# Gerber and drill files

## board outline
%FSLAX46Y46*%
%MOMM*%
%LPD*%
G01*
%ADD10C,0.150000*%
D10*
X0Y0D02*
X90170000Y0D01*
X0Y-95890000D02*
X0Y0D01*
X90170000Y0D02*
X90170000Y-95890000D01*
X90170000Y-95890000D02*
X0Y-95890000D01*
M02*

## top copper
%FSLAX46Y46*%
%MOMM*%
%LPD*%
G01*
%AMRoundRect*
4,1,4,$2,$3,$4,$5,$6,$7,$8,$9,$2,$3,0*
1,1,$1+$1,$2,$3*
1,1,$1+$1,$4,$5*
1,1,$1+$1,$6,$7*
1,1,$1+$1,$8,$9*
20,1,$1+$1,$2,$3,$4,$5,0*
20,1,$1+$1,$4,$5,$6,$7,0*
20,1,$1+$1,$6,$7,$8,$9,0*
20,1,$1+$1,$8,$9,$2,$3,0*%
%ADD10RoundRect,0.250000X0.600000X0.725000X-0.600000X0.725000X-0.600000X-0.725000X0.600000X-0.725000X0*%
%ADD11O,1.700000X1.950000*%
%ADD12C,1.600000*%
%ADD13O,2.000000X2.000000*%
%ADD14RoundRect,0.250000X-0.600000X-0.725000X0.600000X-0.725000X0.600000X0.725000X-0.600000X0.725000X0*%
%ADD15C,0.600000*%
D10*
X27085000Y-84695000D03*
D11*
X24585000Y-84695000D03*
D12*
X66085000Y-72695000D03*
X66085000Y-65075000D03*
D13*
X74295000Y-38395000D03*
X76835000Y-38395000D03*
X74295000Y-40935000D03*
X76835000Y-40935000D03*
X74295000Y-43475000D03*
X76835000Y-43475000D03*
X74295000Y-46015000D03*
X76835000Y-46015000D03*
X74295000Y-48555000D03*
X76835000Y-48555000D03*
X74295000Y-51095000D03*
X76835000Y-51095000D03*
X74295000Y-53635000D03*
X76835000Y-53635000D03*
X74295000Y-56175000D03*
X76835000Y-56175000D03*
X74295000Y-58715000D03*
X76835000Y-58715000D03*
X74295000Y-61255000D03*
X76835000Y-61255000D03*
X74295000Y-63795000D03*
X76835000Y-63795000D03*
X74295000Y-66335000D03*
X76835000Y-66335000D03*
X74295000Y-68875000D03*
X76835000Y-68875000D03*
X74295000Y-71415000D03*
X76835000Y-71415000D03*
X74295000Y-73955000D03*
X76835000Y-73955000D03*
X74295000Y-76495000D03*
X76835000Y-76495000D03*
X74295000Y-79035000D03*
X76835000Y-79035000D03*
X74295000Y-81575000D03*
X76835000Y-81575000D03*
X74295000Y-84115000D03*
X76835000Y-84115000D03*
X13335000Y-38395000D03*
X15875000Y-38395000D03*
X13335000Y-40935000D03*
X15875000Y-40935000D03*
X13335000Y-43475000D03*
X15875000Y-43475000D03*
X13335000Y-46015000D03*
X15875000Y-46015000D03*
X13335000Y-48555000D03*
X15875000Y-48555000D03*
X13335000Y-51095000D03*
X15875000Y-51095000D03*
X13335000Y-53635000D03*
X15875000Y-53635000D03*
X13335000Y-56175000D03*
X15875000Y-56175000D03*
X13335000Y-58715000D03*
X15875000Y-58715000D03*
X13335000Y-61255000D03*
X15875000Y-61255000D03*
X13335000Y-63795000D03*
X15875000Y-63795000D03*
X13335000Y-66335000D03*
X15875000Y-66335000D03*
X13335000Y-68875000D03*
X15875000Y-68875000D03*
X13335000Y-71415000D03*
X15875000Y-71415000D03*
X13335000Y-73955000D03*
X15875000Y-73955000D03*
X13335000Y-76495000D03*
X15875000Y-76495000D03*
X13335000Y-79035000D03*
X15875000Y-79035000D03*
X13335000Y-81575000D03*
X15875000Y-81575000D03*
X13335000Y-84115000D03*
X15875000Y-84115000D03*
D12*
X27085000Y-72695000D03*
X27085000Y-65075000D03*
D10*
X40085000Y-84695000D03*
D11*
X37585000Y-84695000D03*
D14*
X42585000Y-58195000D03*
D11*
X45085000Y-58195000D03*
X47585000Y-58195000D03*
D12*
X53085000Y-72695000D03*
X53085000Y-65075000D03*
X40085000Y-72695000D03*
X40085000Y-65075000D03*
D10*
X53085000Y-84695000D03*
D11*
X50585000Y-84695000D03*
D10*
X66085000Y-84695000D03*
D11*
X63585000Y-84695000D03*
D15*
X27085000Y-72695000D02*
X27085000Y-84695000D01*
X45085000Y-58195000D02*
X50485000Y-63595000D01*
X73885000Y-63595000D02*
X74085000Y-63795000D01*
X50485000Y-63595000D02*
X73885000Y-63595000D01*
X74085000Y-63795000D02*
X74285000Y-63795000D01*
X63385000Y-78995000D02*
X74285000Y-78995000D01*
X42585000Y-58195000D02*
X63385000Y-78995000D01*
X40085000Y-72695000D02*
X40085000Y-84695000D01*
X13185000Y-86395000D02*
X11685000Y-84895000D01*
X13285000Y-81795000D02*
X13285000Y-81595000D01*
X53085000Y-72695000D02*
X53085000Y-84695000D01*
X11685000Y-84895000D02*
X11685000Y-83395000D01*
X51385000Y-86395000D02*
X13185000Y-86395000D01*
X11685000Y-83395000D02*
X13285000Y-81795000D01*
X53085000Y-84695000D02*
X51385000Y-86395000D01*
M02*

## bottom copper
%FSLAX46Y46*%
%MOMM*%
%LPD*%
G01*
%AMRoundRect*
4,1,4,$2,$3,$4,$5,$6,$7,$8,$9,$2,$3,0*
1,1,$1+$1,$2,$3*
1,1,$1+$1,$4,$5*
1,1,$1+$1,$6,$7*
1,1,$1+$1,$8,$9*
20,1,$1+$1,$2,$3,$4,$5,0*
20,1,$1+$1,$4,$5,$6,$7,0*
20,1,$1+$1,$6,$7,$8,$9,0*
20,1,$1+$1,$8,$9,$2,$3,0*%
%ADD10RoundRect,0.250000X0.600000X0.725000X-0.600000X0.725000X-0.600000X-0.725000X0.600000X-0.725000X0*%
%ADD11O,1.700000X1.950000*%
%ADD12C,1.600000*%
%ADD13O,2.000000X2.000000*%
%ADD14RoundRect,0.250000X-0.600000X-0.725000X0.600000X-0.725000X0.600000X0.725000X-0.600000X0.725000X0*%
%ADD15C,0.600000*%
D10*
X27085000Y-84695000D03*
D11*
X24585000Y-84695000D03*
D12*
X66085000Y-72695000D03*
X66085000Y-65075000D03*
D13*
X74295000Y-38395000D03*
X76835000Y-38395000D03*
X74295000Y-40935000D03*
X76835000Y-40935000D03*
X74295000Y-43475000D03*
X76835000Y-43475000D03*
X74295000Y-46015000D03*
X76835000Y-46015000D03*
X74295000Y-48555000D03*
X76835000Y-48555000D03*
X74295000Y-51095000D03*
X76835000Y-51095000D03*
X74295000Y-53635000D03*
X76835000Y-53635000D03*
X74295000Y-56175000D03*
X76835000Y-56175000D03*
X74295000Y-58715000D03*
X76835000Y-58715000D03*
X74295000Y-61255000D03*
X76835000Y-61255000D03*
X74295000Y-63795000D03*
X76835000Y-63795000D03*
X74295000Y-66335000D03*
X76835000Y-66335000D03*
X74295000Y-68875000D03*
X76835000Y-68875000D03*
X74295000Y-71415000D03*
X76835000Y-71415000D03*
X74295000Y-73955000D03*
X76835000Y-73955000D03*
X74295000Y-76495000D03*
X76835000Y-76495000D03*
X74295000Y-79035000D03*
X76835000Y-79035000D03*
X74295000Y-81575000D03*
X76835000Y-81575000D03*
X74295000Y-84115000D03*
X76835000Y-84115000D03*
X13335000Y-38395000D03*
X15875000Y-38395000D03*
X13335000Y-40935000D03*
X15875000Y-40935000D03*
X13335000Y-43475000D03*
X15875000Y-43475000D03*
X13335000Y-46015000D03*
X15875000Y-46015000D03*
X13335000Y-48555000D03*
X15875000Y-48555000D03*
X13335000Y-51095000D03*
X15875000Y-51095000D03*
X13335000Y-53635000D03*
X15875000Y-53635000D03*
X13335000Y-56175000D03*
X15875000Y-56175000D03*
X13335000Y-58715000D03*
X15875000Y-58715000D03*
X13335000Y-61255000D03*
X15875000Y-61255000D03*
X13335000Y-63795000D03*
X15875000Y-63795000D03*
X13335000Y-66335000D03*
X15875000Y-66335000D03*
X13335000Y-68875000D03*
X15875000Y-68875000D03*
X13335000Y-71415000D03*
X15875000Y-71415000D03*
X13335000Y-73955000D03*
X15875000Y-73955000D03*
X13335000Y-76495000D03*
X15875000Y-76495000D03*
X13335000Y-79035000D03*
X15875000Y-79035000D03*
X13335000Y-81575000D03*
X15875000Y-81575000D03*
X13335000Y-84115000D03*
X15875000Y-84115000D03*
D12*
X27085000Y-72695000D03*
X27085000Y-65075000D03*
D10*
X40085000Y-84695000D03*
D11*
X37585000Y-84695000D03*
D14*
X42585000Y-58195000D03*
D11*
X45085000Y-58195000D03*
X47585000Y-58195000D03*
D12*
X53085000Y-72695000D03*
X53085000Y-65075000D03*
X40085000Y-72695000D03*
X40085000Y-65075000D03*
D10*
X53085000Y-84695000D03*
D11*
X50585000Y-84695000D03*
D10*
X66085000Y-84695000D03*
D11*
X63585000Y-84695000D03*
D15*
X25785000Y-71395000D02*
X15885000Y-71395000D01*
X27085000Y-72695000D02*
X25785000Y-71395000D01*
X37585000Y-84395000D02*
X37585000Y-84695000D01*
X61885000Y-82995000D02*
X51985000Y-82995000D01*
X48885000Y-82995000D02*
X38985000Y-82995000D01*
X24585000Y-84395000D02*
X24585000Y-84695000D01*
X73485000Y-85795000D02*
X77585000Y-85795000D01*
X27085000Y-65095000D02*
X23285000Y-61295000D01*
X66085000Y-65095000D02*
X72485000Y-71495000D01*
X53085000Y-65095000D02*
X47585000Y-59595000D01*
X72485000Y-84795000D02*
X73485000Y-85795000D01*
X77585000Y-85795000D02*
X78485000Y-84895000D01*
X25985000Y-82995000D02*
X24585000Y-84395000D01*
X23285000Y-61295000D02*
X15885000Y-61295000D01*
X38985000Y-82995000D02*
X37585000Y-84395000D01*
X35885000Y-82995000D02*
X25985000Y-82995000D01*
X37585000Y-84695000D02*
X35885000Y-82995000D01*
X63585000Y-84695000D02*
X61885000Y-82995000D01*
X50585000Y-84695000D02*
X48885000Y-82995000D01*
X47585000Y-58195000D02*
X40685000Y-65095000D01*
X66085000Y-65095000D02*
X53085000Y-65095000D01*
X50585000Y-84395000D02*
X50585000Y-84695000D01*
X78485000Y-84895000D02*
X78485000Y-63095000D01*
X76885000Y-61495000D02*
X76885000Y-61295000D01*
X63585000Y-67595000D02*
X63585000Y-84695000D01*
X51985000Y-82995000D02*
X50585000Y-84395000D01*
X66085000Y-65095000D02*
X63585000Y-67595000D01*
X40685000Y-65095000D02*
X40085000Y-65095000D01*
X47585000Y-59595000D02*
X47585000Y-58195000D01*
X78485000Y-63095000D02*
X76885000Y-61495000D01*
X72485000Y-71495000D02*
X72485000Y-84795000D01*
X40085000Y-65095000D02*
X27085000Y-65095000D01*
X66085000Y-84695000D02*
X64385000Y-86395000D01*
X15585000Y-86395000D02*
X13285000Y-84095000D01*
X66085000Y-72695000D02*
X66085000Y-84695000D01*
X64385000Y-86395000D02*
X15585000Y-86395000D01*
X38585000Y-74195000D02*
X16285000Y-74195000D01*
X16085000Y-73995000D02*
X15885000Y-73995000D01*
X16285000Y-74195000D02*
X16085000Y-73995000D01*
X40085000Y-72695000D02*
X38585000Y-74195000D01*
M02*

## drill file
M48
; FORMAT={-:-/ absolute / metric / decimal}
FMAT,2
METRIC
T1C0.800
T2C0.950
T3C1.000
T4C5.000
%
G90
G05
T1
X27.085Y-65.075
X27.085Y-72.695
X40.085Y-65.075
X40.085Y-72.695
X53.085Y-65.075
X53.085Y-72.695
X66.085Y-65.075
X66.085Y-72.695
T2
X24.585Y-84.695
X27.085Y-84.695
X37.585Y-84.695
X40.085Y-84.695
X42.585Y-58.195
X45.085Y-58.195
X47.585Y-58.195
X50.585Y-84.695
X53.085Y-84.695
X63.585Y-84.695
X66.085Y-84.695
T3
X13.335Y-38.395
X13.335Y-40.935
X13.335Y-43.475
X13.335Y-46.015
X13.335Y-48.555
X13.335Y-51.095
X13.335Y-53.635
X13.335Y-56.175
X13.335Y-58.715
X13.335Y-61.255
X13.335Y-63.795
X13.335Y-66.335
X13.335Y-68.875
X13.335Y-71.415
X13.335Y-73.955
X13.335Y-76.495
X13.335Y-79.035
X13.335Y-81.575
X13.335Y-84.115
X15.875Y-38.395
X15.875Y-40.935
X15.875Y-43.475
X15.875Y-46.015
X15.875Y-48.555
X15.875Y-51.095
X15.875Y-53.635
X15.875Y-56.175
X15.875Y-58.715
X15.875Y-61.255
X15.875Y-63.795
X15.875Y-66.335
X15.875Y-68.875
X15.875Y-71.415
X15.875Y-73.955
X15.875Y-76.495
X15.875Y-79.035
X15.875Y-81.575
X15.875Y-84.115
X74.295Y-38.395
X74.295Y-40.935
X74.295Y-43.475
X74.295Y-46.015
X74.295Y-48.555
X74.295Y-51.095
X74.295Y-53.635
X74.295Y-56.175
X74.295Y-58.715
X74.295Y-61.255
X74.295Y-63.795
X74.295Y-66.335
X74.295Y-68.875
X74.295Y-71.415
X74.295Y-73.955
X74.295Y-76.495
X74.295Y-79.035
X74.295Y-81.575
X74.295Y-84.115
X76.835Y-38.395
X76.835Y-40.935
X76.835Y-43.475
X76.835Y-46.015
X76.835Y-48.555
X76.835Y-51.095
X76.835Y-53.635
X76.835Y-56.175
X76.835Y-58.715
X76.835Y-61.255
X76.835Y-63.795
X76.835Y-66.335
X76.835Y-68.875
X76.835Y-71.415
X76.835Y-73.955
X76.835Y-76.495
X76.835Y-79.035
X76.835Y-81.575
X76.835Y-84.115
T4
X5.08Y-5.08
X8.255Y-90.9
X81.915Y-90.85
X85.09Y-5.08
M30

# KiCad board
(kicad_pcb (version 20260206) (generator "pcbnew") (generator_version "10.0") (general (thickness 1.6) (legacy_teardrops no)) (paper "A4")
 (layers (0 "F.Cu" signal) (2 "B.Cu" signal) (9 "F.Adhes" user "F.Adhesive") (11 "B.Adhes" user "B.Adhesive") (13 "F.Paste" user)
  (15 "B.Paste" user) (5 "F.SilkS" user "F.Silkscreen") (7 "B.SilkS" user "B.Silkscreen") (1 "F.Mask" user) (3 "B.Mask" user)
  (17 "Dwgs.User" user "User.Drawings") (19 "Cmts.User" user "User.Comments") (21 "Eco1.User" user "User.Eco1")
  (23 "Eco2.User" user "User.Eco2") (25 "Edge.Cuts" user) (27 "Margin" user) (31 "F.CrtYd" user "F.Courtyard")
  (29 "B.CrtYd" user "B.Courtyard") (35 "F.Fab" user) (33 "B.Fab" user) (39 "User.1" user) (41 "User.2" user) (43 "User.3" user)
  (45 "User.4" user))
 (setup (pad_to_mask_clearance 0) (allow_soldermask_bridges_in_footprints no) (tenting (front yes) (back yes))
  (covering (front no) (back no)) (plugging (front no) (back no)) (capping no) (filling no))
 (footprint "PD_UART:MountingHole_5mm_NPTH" (layer "F.Cu") (at 8.255 90.9)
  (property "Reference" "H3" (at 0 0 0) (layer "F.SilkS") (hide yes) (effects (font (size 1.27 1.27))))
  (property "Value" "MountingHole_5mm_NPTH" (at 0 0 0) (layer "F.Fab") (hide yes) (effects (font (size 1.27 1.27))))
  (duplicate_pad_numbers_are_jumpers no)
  (pad "" np_thru_hole circle (at 0 0) (size 5 5) (drill 5) (layers "*.Cu")))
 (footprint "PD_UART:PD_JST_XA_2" (layer "F.Cu") (at 27.085 84.695 180)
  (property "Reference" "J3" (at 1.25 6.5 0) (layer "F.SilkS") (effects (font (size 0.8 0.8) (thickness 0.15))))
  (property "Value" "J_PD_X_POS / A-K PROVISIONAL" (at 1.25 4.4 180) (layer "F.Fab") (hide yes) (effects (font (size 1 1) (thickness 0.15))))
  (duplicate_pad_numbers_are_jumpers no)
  (pad "1" thru_hole roundrect (at 0 0 180) (size 1.7 1.95) (drill 0.95) (layers "*.Cu") (remove_unused_layers no)
   (roundrect_rratio 0.147059) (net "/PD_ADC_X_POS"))
  (pad "2" thru_hole oval (at 2.5 0 180) (size 1.7 1.95) (drill 0.95) (layers "*.Cu") (remove_unused_layers no) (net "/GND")))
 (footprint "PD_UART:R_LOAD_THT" (layer "F.Cu") (at 66.085 72.695 90)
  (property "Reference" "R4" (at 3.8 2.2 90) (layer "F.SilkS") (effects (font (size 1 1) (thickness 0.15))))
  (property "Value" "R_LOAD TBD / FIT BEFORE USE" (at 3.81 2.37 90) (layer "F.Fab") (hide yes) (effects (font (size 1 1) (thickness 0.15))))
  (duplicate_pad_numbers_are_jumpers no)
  (pad "1" thru_hole circle (at 0 0 90) (size 1.6 1.6) (drill 0.8) (layers "*.Cu") (remove_unused_layers no) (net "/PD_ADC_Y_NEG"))
  (pad "2" thru_hole circle (at 7.62 0 90) (size 1.6 1.6) (drill 0.8) (layers "*.Cu") (remove_unused_layers no) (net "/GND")))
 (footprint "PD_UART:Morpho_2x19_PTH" (layer "F.Cu") (at 74.295 38.395)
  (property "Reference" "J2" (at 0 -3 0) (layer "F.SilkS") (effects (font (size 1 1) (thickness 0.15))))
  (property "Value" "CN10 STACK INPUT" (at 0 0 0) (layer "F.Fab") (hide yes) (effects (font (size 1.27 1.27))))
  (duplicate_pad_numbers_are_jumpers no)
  (pad "1" thru_hole oval (at 0 0) (size 2 2) (drill 1) (layers "*.Cu") (remove_unused_layers no) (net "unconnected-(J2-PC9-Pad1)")
   (thermal_bridge_angle 45))
  (pad "2" thru_hole oval (at 2.54 0) (size 2 2) (drill 1) (layers "*.Cu") (remove_unused_layers no) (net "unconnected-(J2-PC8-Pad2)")
   (thermal_bridge_angle 45))
  (pad "3" thru_hole oval (at 0 2.54) (size 2 2) (drill 1) (layers "*.Cu") (remove_unused_layers no) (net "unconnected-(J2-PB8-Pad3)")
   (thermal_bridge_angle 45))
  (pad "4" thru_hole oval (at 2.54 2.54) (size 2 2) (drill 1) (layers "*.Cu") (remove_unused_layers no) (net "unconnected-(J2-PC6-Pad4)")
   (thermal_bridge_angle 45))
  (pad "5" thru_hole oval (at 0 5.08) (size 2 2) (drill 1) (layers "*.Cu") (remove_unused_layers no) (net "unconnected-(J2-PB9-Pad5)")
   (thermal_bridge_angle 45))
  (pad "6" thru_hole oval (at 2.54 5.08) (size 2 2) (drill 1) (layers "*.Cu") (remove_unused_layers no) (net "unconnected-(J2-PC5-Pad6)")
   (thermal_bridge_angle 45))
  (pad "7" thru_hole oval (at 0 7.62) (size 2 2) (drill 1) (layers "*.Cu") (remove_unused_layers no) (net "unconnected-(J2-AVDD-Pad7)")
   (thermal_bridge_angle 45))
  (pad "8" thru_hole oval (at 2.54 7.62) (size 2 2) (drill 1) (layers "*.Cu") (remove_unused_layers no) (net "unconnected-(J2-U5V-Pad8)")
   (thermal_bridge_angle 45))
  (pad "9" thru_hole oval (at 0 10.16) (size 2 2) (drill 1) (layers "*.Cu") (remove_unused_layers no) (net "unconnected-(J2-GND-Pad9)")
   (thermal_bridge_angle 45))
  (pad "10" thru_hole oval (at 2.54 10.16) (size 2 2) (drill 1) (layers "*.Cu") (remove_unused_layers no) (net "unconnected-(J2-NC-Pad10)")
   (thermal_bridge_angle 45))
  (pad "11" thru_hole oval (at 0 12.7) (size 2 2) (drill 1) (layers "*.Cu") (remove_unused_layers no) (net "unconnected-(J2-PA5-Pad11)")
   (thermal_bridge_angle 45))
  (pad "12" thru_hole oval (at 2.54 12.7) (size 2 2) (drill 1) (layers "*.Cu") (remove_unused_layers no) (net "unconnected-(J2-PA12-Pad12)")
   (thermal_bridge_angle 45))
  (pad "13" thru_hole oval (at 0 15.24) (size 2 2) (drill 1) (layers "*.Cu") (remove_unused_layers no) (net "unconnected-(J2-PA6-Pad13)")
   (thermal_bridge_angle 45))
  (pad "14" thru_hole oval (at 2.54 15.24) (size 2 2) (drill 1) (layers "*.Cu") (remove_unused_layers no)
   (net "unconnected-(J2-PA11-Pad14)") (thermal_bridge_angle 45))
  (pad "15" thru_hole oval (at 0 17.78) (size 2 2) (drill 1) (layers "*.Cu") (remove_unused_layers no) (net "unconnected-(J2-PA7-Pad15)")
   (thermal_bridge_angle 45))
  (pad "16" thru_hole oval (at 2.54 17.78) (size 2 2) (drill 1) (layers "*.Cu") (remove_unused_layers no)
   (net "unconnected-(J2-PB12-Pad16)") (thermal_bridge_angle 45))
  (pad "17" thru_hole oval (at 0 20.32) (size 2 2) (drill 1) (layers "*.Cu") (remove_unused_layers no) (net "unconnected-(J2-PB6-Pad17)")
   (thermal_bridge_angle 45))
  (pad "18" thru_hole oval (at 2.54 20.32) (size 2 2) (drill 1) (layers "*.Cu") (remove_unused_layers no)
   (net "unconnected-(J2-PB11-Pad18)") (thermal_bridge_angle 45))
  (pad "19" thru_hole oval (at 0 22.86) (size 2 2) (drill 1) (layers "*.Cu") (remove_unused_layers no) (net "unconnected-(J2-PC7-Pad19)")
   (thermal_bridge_angle 45))
  (pad "20" thru_hole oval (at 2.54 22.86) (size 2 2) (drill 1) (layers "*.Cu") (remove_unused_layers no) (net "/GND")
   (thermal_bridge_angle 45))
  (pad "21" thru_hole oval (at 0 25.4) (size 2 2) (drill 1) (layers "*.Cu") (remove_unused_layers no) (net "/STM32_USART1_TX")
   (thermal_bridge_angle 45))
  (pad "22" thru_hole oval (at 2.54 25.4) (size 2 2) (drill 1) (layers "*.Cu") (remove_unused_layers no) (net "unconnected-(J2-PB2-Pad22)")
   (thermal_bridge_angle 45))
  (pad "23" thru_hole oval (at 0 27.94) (size 2 2) (drill 1) (layers "*.Cu") (remove_unused_layers no) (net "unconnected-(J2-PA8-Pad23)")
   (thermal_bridge_angle 45))
  (pad "24" thru_hole oval (at 2.54 27.94) (size 2 2) (drill 1) (layers "*.Cu") (remove_unused_layers no) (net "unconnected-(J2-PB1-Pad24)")
   (thermal_bridge_angle 45))
  (pad "25" thru_hole oval (at 0 30.48) (size 2 2) (drill 1) (layers "*.Cu") (remove_unused_layers no) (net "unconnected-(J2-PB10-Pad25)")
   (thermal_bridge_angle 45))
  (pad "26" thru_hole oval (at 2.54 30.48) (size 2 2) (drill 1) (layers "*.Cu") (remove_unused_layers no)
   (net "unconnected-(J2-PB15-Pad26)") (thermal_bridge_angle 45))
  (pad "27" thru_hole oval (at 0 33.02) (size 2 2) (drill 1) (layers "*.Cu") (remove_unused_layers no) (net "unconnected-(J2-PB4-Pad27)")
   (thermal_bridge_angle 45))
  (pad "28" thru_hole oval (at 2.54 33.02) (size 2 2) (drill 1) (layers "*.Cu") (remove_unused_layers no)
   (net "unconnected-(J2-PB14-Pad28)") (thermal_bridge_angle 45))
  (pad "29" thru_hole oval (at 0 35.56) (size 2 2) (drill 1) (layers "*.Cu") (remove_unused_layers no) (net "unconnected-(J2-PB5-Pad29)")
   (thermal_bridge_angle 45))
  (pad "30" thru_hole oval (at 2.54 35.56) (size 2 2) (drill 1) (layers "*.Cu") (remove_unused_layers no)
   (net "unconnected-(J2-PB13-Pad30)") (thermal_bridge_angle 45))
  (pad "31" thru_hole oval (at 0 38.1) (size 2 2) (drill 1) (layers "*.Cu") (remove_unused_layers no) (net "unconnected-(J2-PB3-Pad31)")
   (thermal_bridge_angle 45))
  (pad "32" thru_hole oval (at 2.54 38.1) (size 2 2) (drill 1) (layers "*.Cu") (remove_unused_layers no) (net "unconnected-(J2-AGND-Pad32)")
   (thermal_bridge_angle 45))
  (pad "33" thru_hole oval (at 0 40.64) (size 2 2) (drill 1) (layers "*.Cu") (remove_unused_layers no) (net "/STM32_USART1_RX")
   (thermal_bridge_angle 45))
  (pad "34" thru_hole oval (at 2.54 40.64) (size 2 2) (drill 1) (layers "*.Cu") (remove_unused_layers no) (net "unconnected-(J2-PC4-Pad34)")
   (thermal_bridge_angle 45))
  (pad "35" thru_hole oval (at 0 43.18) (size 2 2) (drill 1) (layers "*.Cu") (remove_unused_layers no) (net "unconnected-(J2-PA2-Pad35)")
   (thermal_bridge_angle 45))
  (pad "36" thru_hole oval (at 2.54 43.18) (size 2 2) (drill 1) (layers "*.Cu") (remove_unused_layers no) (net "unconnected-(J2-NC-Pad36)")
   (thermal_bridge_angle 45))
  (pad "37" thru_hole oval (at 0 45.72) (size 2 2) (drill 1) (layers "*.Cu") (remove_unused_layers no) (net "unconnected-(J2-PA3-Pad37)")
   (thermal_bridge_angle 45))
  (pad "38" thru_hole oval (at 2.54 45.72) (size 2 2) (drill 1) (layers "*.Cu") (remove_unused_layers no) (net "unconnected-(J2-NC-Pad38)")
   (thermal_bridge_angle 45)))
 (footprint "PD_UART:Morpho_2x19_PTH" (layer "F.Cu") (at 13.335 38.395)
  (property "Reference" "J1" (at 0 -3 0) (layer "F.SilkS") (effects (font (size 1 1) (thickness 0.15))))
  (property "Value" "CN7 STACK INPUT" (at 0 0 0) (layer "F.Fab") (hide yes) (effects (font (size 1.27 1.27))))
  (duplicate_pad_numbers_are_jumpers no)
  (pad "1" thru_hole oval (at 0 0) (size 2 2) (drill 1) (layers "*.Cu") (remove_unused_layers no) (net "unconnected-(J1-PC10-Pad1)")
   (thermal_bridge_angle 45))
  (pad "2" thru_hole oval (at 2.54 0) (size 2 2) (drill 1) (layers "*.Cu") (remove_unused_layers no) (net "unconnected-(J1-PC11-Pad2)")
   (thermal_bridge_angle 45))
  (pad "3" thru_hole oval (at 0 2.54) (size 2 2) (drill 1) (layers "*.Cu") (remove_unused_layers no) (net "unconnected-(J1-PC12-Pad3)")
   (thermal_bridge_angle 45))
  (pad "4" thru_hole oval (at 2.54 2.54) (size 2 2) (drill 1) (layers "*.Cu") (remove_unused_layers no) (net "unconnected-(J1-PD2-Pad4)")
   (thermal_bridge_angle 45))
  (pad "5" thru_hole oval (at 0 5.08) (size 2 2) (drill 1) (layers "*.Cu") (remove_unused_layers no) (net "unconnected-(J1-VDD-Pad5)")
   (thermal_bridge_angle 45))
  (pad "6" thru_hole oval (at 2.54 5.08) (size 2 2) (drill 1) (layers "*.Cu") (remove_unused_layers no) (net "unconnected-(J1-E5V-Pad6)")
   (thermal_bridge_angle 45))
  (pad "7" thru_hole oval (at 0 7.62) (size 2 2) (drill 1) (layers "*.Cu") (remove_unused_layers no) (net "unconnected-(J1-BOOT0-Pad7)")
   (thermal_bridge_angle 45))
  (pad "8" thru_hole oval (at 2.54 7.62) (size 2 2) (drill 1) (layers "*.Cu") (remove_unused_layers no) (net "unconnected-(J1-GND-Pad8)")
   (thermal_bridge_angle 45))
  (pad "9" thru_hole oval (at 0 10.16) (size 2 2) (drill 1) (layers "*.Cu") (remove_unused_layers no) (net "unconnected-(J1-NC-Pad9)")
   (thermal_bridge_angle 45))
  (pad "10" thru_hole oval (at 2.54 10.16) (size 2 2) (drill 1) (layers "*.Cu") (remove_unused_layers no) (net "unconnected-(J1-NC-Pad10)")
   (thermal_bridge_angle 45))
  (pad "11" thru_hole oval (at 0 12.7) (size 2 2) (drill 1) (layers "*.Cu") (remove_unused_layers no) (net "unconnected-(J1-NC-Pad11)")
   (thermal_bridge_angle 45))
  (pad "12" thru_hole oval (at 2.54 12.7) (size 2 2) (drill 1) (layers "*.Cu") (remove_unused_layers no)
   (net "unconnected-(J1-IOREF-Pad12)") (thermal_bridge_angle 45))
  (pad "13" thru_hole oval (at 0 15.24) (size 2 2) (drill 1) (layers "*.Cu") (remove_unused_layers no) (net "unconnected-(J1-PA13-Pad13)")
   (thermal_bridge_angle 45))
  (pad "14" thru_hole oval (at 2.54 15.24) (size 2 2) (drill 1) (layers "*.Cu") (remove_unused_layers no)
   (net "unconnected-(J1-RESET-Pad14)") (thermal_bridge_angle 45))
  (pad "15" thru_hole oval (at 0 17.78) (size 2 2) (drill 1) (layers "*.Cu") (remove_unused_layers no) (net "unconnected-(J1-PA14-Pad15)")
   (thermal_bridge_angle 45))
  (pad "16" thru_hole oval (at 2.54 17.78) (size 2 2) (drill 1) (layers "*.Cu") (remove_unused_layers no) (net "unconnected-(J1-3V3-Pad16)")
   (thermal_bridge_angle 45))
  (pad "17" thru_hole oval (at 0 20.32) (size 2 2) (drill 1) (layers "*.Cu") (remove_unused_layers no) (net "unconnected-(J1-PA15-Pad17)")
   (thermal_bridge_angle 45))
  (pad "18" thru_hole oval (at 2.54 20.32) (size 2 2) (drill 1) (layers "*.Cu") (remove_unused_layers no) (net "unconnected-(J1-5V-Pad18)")
   (thermal_bridge_angle 45))
  (pad "19" thru_hole oval (at 0 22.86) (size 2 2) (drill 1) (layers "*.Cu") (remove_unused_layers no) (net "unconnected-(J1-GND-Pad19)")
   (thermal_bridge_angle 45))
  (pad "20" thru_hole oval (at 2.54 22.86) (size 2 2) (drill 1) (layers "*.Cu") (remove_unused_layers no) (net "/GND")
   (thermal_bridge_angle 45))
  (pad "21" thru_hole oval (at 0 25.4) (size 2 2) (drill 1) (layers "*.Cu") (remove_unused_layers no) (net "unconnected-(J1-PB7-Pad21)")
   (thermal_bridge_angle 45))
  (pad "22" thru_hole oval (at 2.54 25.4) (size 2 2) (drill 1) (layers "*.Cu") (remove_unused_layers no) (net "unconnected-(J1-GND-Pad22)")
   (thermal_bridge_angle 45))
  (pad "23" thru_hole oval (at 0 27.94) (size 2 2) (drill 1) (layers "*.Cu") (remove_unused_layers no) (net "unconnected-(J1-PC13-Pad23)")
   (thermal_bridge_angle 45))
  (pad "24" thru_hole oval (at 2.54 27.94) (size 2 2) (drill 1) (layers "*.Cu") (remove_unused_layers no) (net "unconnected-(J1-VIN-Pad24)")
   (thermal_bridge_angle 45))
  (pad "25" thru_hole oval (at 0 30.48) (size 2 2) (drill 1) (layers "*.Cu") (remove_unused_layers no) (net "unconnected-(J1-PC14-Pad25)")
   (thermal_bridge_angle 45))
  (pad "26" thru_hole oval (at 2.54 30.48) (size 2 2) (drill 1) (layers "*.Cu") (remove_unused_layers no) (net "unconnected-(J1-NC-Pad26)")
   (thermal_bridge_angle 45))
  (pad "27" thru_hole oval (at 0 33.02) (size 2 2) (drill 1) (layers "*.Cu") (remove_unused_layers no) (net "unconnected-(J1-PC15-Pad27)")
   (thermal_bridge_angle 45))
  (pad "28" thru_hole oval (at 2.54 33.02) (size 2 2) (drill 1) (layers "*.Cu") (remove_unused_layers no) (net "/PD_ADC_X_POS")
   (thermal_bridge_angle 45))
  (pad "29" thru_hole oval (at 0 35.56) (size 2 2) (drill 1) (layers "*.Cu") (remove_unused_layers no) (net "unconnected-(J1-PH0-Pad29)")
   (thermal_bridge_angle 45))
  (pad "30" thru_hole oval (at 2.54 35.56) (size 2 2) (drill 1) (layers "*.Cu") (remove_unused_layers no) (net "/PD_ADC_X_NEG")
   (thermal_bridge_angle 45))
  (pad "31" thru_hole oval (at 0 38.1) (size 2 2) (drill 1) (layers "*.Cu") (remove_unused_layers no) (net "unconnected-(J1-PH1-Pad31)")
   (thermal_bridge_angle 45))
  (pad "32" thru_hole oval (at 2.54 38.1) (size 2 2) (drill 1) (layers "*.Cu") (remove_unused_layers no) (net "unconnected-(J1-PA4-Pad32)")
   (thermal_bridge_angle 45))
  (pad "33" thru_hole oval (at 0 40.64) (size 2 2) (drill 1) (layers "*.Cu") (remove_unused_layers no) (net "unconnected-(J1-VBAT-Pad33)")
   (thermal_bridge_angle 45))
  (pad "34" thru_hole oval (at 2.54 40.64) (size 2 2) (drill 1) (layers "*.Cu") (remove_unused_layers no) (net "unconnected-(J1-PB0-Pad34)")
   (thermal_bridge_angle 45))
  (pad "35" thru_hole oval (at 0 43.18) (size 2 2) (drill 1) (layers "*.Cu") (remove_unused_layers no) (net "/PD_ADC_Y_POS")
   (thermal_bridge_angle 45))
  (pad "36" thru_hole oval (at 2.54 43.18) (size 2 2) (drill 1) (layers "*.Cu") (remove_unused_layers no)
   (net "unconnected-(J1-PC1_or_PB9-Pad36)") (thermal_bridge_angle 45))
  (pad "37" thru_hole oval (at 0 45.72) (size 2 2) (drill 1) (layers "*.Cu") (remove_unused_layers no) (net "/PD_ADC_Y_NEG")
   (thermal_bridge_angle 45))
  (pad "38" thru_hole oval (at 2.54 45.72) (size 2 2) (drill 1) (layers "*.Cu") (remove_unused_layers no) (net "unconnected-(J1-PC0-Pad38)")
   (thermal_bridge_angle 45)))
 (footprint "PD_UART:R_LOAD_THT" (layer "F.Cu") (at 27.085 72.695 90)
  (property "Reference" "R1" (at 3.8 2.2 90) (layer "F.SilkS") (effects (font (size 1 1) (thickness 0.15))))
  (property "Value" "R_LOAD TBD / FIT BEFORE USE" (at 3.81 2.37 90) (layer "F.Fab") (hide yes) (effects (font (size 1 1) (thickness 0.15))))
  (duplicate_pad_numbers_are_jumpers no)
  (pad "1" thru_hole circle (at 0 0 90) (size 1.6 1.6) (drill 0.8) (layers "*.Cu") (remove_unused_layers no) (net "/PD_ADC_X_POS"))
  (pad "2" thru_hole circle (at 7.62 0 90) (size 1.6 1.6) (drill 0.8) (layers "*.Cu") (remove_unused_layers no) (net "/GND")))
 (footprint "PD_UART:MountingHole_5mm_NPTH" (layer "F.Cu") (at 81.915 90.85)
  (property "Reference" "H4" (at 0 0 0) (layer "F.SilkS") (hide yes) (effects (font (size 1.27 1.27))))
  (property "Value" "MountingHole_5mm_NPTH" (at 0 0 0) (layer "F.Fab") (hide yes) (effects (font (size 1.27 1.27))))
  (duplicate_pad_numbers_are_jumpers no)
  (pad "" np_thru_hole circle (at 0 0) (size 5 5) (drill 5) (layers "*.Cu")))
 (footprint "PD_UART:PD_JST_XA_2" (layer "F.Cu") (at 40.085 84.695 180)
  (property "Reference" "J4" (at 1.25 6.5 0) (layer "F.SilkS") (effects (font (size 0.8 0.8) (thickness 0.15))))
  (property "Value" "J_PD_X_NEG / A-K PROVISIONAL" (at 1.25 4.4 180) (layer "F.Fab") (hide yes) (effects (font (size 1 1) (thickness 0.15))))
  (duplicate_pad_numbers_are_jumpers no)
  (pad "1" thru_hole roundrect (at 0 0 180) (size 1.7 1.95) (drill 0.95) (layers "*.Cu") (remove_unused_layers no)
   (roundrect_rratio 0.147059) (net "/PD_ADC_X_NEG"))
  (pad "2" thru_hole oval (at 2.5 0 180) (size 1.7 1.95) (drill 0.95) (layers "*.Cu") (remove_unused_layers no) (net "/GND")))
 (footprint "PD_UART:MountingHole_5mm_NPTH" (layer "F.Cu") (at 85.09 5.08)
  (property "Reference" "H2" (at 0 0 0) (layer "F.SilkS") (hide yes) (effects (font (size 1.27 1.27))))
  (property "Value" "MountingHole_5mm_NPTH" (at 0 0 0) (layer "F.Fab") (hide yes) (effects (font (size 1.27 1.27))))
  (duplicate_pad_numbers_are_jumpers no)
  (pad "" np_thru_hole circle (at 0 0) (size 5 5) (drill 5) (layers "*.Cu")))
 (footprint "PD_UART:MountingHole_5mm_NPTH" (layer "F.Cu") (at 5.08 5.08)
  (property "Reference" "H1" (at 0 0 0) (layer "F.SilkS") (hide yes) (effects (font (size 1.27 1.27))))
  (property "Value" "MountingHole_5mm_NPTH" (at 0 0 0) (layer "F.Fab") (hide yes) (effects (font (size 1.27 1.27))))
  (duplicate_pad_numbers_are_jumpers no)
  (pad "" np_thru_hole circle (at 0 0) (size 5 5) (drill 5) (layers "*.Cu")))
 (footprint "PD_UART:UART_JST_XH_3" (layer "F.Cu") (at 42.585 58.195)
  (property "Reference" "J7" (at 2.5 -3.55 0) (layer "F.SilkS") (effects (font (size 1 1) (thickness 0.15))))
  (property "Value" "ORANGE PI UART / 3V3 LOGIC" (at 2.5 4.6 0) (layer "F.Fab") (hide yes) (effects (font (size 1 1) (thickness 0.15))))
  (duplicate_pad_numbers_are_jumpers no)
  (pad "1" thru_hole roundrect (at 0 0) (size 1.7 1.95) (drill 0.95) (layers "*.Cu") (remove_unused_layers no) (roundrect_rratio 0.147059)
   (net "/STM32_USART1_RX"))
  (pad "2" thru_hole oval (at 2.5 0) (size 1.7 1.95) (drill 0.95) (layers "*.Cu") (remove_unused_layers no) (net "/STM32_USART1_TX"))
  (pad "3" thru_hole oval (at 5 0) (size 1.7 1.95) (drill 0.95) (layers "*.Cu") (remove_unused_layers no) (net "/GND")))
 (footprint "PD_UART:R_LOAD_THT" (layer "F.Cu") (at 53.085 72.695 90)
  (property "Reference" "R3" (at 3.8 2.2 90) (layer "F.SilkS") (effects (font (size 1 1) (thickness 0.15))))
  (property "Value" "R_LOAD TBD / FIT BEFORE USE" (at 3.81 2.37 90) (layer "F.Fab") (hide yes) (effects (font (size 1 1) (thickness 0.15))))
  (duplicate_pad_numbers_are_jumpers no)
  (pad "1" thru_hole circle (at 0 0 90) (size 1.6 1.6) (drill 0.8) (layers "*.Cu") (remove_unused_layers no) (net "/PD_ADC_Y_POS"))
  (pad "2" thru_hole circle (at 7.62 0 90) (size 1.6 1.6) (drill 0.8) (layers "*.Cu") (remove_unused_layers no) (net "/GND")))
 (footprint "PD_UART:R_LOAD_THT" (layer "F.Cu") (at 40.085 72.695 90)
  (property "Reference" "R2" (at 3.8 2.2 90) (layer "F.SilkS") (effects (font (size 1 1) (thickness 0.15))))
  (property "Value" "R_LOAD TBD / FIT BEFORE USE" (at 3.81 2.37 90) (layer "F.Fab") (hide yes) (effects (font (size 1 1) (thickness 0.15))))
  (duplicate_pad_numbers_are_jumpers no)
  (pad "1" thru_hole circle (at 0 0 90) (size 1.6 1.6) (drill 0.8) (layers "*.Cu") (remove_unused_layers no) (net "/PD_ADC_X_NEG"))
  (pad "2" thru_hole circle (at 7.62 0 90) (size 1.6 1.6) (drill 0.8) (layers "*.Cu") (remove_unused_layers no) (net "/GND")))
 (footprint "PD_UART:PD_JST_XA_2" (layer "F.Cu") (at 53.085 84.695 180)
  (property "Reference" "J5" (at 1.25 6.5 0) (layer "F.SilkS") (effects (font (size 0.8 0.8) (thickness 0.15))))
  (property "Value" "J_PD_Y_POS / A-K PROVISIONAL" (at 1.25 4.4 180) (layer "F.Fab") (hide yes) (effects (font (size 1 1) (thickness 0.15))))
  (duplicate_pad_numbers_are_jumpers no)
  (pad "1" thru_hole roundrect (at 0 0 180) (size 1.7 1.95) (drill 0.95) (layers "*.Cu") (remove_unused_layers no)
   (roundrect_rratio 0.147059) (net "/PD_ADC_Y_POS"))
  (pad "2" thru_hole oval (at 2.5 0 180) (size 1.7 1.95) (drill 0.95) (layers "*.Cu") (remove_unused_layers no) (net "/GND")))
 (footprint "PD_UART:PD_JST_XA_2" (layer "F.Cu") (at 66.085 84.695 180)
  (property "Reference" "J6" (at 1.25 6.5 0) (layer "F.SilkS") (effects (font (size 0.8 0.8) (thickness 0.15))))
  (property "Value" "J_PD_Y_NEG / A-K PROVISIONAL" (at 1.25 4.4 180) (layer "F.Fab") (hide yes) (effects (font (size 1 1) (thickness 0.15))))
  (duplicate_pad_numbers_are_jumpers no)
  (pad "1" thru_hole roundrect (at 0 0 180) (size 1.7 1.95) (drill 0.95) (layers "*.Cu") (remove_unused_layers no)
   (roundrect_rratio 0.147059) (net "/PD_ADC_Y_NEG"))
  (pad "2" thru_hole oval (at 2.5 0 180) (size 1.7 1.95) (drill 0.95) (layers "*.Cu") (remove_unused_layers no) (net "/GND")))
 (gr_line (start 0 0) (end 90.17 0) (stroke (width 0.15) (type default)) (layer "Edge.Cuts"))
 (gr_line (start 0 95.89) (end 0 0) (stroke (width 0.15) (type default)) (layer "Edge.Cuts"))
 (gr_line (start 90.17 0) (end 90.17 95.89) (stroke (width 0.15) (type default)) (layer "Edge.Cuts"))
 (gr_line (start 90.17 95.89) (end 0 95.89) (stroke (width 0.15) (type default)) (layer "Edge.Cuts"))
 (segment (start 27.085 72.695) (end 27.085 84.695) (width 0.6) (layer "F.Cu") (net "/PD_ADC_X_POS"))
 (segment (start 25.785 71.395) (end 15.885 71.395) (width 0.6) (layer "B.Cu") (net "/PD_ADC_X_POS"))
 (segment (start 27.085 72.695) (end 25.785 71.395) (width 0.6) (layer "B.Cu") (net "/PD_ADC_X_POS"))
 (segment (start 37.585 84.395) (end 37.585 84.695) (width 0.6) (layer "B.Cu") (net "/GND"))
 (segment (start 61.885 82.995) (end 51.985 82.995) (width 0.6) (layer "B.Cu") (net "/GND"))
 (segment (start 48.885 82.995) (end 38.985 82.995) (width 0.6) (layer "B.Cu") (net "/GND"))
 (segment (start 24.585 84.395) (end 24.585 84.695) (width 0.6) (layer "B.Cu") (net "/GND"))
 (segment (start 73.485 85.795) (end 77.585 85.795) (width 0.6) (layer "B.Cu") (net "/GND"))
 (segment (start 27.085 65.095) (end 23.285 61.295) (width 0.6) (layer "B.Cu") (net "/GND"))
 (segment (start 66.085 65.095) (end 72.485 71.495) (width 0.6) (layer "B.Cu") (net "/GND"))
 (segment (start 53.085 65.095) (end 47.585 59.595) (width 0.6) (layer "B.Cu") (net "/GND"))
 (segment (start 72.485 84.795) (end 73.485 85.795) (width 0.6) (layer "B.Cu") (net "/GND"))
 (segment (start 77.585 85.795) (end 78.485 84.895) (width 0.6) (layer "B.Cu") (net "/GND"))
 (segment (start 25.985 82.995) (end 24.585 84.395) (width 0.6) (layer "B.Cu") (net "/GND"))
 (segment (start 23.285 61.295) (end 15.885 61.295) (width 0.6) (layer "B.Cu") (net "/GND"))
 (segment (start 38.985 82.995) (end 37.585 84.395) (width 0.6) (layer "B.Cu") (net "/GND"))
 (segment (start 35.885 82.995) (end 25.985 82.995) (width 0.6) (layer "B.Cu") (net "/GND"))
 (segment (start 37.585 84.695) (end 35.885 82.995) (width 0.6) (layer "B.Cu") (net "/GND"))
 (segment (start 63.585 84.695) (end 61.885 82.995) (width 0.6) (layer "B.Cu") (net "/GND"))
 (segment (start 50.585 84.695) (end 48.885 82.995) (width 0.6) (layer "B.Cu") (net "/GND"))
 (segment (start 47.585 58.195) (end 40.685 65.095) (width 0.6) (layer "B.Cu") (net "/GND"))
 (segment (start 66.085 65.095) (end 53.085 65.095) (width 0.6) (layer "B.Cu") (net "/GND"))
 (segment (start 50.585 84.395) (end 50.585 84.695) (width 0.6) (layer "B.Cu") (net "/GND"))
 (segment (start 78.485 84.895) (end 78.485 63.095) (width 0.6) (layer "B.Cu") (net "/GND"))
 (segment (start 76.885 61.495) (end 76.885 61.295) (width 0.6) (layer "B.Cu") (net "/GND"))
 (segment (start 63.585 67.595) (end 63.585 84.695) (width 0.6) (layer "B.Cu") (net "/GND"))
 (segment (start 51.985 82.995) (end 50.585 84.395) (width 0.6) (layer "B.Cu") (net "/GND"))
 (segment (start 66.085 65.095) (end 63.585 67.595) (width 0.6) (layer "B.Cu") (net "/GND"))
 (segment (start 40.685 65.095) (end 40.085 65.095) (width 0.6) (layer "B.Cu") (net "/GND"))
 (segment (start 47.585 59.595) (end 47.585 58.195) (width 0.6) (layer "B.Cu") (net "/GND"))
 (segment (start 78.485 63.095) (end 76.885 61.495) (width 0.6) (layer "B.Cu") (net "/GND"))
 (segment (start 72.485 71.495) (end 72.485 84.795) (width 0.6) (layer "B.Cu") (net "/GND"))
 (segment (start 40.085 65.095) (end 27.085 65.095) (width 0.6) (layer "B.Cu") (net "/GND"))
 (segment (start 66.085 84.695) (end 64.385 86.395) (width 0.6) (layer "B.Cu") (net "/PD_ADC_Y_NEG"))
 (segment (start 15.585 86.395) (end 13.285 84.095) (width 0.6) (layer "B.Cu") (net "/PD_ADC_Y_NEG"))
 (segment (start 66.085 72.695) (end 66.085 84.695) (width 0.6) (layer "B.Cu") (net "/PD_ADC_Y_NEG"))
 (segment (start 64.385 86.395) (end 15.585 86.395) (width 0.6) (layer "B.Cu") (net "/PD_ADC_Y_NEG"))
 (segment (start 45.085 58.195) (end 50.485 63.595) (width 0.6) (layer "F.Cu") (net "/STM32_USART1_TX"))
 (segment (start 73.885 63.595) (end 74.085 63.795) (width 0.6) (layer "F.Cu") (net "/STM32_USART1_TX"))
 (segment (start 50.485 63.595) (end 73.885 63.595) (width 0.6) (layer "F.Cu") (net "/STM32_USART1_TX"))
 (segment (start 74.085 63.795) (end 74.285 63.795) (width 0.6) (layer "F.Cu") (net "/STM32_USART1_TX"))
 (segment (start 63.385 78.995) (end 74.285 78.995) (width 0.6) (layer "F.Cu") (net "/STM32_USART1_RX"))
 (segment (start 42.585 58.195) (end 63.385 78.995) (width 0.6) (layer "F.Cu") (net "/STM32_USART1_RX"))
 (segment (start 40.085 72.695) (end 40.085 84.695) (width 0.6) (layer "F.Cu") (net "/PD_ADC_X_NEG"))
 (segment (start 38.585 74.195) (end 16.285 74.195) (width 0.6) (layer "B.Cu") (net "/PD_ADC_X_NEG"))
 (segment (start 16.085 73.995) (end 15.885 73.995) (width 0.6) (layer "B.Cu") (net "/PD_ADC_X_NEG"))
 (segment (start 16.285 74.195) (end 16.085 73.995) (width 0.6) (layer "B.Cu") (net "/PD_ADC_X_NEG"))
 (segment (start 40.085 72.695) (end 38.585 74.195) (width 0.6) (layer "B.Cu") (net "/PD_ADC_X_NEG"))
 (segment (start 13.185 86.395) (end 11.685 84.895) (width 0.6) (layer "F.Cu") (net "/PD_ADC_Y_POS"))
 (segment (start 13.285 81.795) (end 13.285 81.595) (width 0.6) (layer "F.Cu") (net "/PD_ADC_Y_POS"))
 (segment (start 53.085 72.695) (end 53.085 84.695) (width 0.6) (layer "F.Cu") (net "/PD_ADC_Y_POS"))
 (segment (start 11.685 84.895) (end 11.685 83.395) (width 0.6) (layer "F.Cu") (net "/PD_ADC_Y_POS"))
 (segment (start 51.385 86.395) (end 13.185 86.395) (width 0.6) (layer "F.Cu") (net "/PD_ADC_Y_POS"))
 (segment (start 11.685 83.395) (end 13.285 81.795) (width 0.6) (layer "F.Cu") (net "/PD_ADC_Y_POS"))
 (segment (start 53.085 84.695) (end 51.385 86.395) (width 0.6) (layer "F.Cu") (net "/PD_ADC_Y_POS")))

